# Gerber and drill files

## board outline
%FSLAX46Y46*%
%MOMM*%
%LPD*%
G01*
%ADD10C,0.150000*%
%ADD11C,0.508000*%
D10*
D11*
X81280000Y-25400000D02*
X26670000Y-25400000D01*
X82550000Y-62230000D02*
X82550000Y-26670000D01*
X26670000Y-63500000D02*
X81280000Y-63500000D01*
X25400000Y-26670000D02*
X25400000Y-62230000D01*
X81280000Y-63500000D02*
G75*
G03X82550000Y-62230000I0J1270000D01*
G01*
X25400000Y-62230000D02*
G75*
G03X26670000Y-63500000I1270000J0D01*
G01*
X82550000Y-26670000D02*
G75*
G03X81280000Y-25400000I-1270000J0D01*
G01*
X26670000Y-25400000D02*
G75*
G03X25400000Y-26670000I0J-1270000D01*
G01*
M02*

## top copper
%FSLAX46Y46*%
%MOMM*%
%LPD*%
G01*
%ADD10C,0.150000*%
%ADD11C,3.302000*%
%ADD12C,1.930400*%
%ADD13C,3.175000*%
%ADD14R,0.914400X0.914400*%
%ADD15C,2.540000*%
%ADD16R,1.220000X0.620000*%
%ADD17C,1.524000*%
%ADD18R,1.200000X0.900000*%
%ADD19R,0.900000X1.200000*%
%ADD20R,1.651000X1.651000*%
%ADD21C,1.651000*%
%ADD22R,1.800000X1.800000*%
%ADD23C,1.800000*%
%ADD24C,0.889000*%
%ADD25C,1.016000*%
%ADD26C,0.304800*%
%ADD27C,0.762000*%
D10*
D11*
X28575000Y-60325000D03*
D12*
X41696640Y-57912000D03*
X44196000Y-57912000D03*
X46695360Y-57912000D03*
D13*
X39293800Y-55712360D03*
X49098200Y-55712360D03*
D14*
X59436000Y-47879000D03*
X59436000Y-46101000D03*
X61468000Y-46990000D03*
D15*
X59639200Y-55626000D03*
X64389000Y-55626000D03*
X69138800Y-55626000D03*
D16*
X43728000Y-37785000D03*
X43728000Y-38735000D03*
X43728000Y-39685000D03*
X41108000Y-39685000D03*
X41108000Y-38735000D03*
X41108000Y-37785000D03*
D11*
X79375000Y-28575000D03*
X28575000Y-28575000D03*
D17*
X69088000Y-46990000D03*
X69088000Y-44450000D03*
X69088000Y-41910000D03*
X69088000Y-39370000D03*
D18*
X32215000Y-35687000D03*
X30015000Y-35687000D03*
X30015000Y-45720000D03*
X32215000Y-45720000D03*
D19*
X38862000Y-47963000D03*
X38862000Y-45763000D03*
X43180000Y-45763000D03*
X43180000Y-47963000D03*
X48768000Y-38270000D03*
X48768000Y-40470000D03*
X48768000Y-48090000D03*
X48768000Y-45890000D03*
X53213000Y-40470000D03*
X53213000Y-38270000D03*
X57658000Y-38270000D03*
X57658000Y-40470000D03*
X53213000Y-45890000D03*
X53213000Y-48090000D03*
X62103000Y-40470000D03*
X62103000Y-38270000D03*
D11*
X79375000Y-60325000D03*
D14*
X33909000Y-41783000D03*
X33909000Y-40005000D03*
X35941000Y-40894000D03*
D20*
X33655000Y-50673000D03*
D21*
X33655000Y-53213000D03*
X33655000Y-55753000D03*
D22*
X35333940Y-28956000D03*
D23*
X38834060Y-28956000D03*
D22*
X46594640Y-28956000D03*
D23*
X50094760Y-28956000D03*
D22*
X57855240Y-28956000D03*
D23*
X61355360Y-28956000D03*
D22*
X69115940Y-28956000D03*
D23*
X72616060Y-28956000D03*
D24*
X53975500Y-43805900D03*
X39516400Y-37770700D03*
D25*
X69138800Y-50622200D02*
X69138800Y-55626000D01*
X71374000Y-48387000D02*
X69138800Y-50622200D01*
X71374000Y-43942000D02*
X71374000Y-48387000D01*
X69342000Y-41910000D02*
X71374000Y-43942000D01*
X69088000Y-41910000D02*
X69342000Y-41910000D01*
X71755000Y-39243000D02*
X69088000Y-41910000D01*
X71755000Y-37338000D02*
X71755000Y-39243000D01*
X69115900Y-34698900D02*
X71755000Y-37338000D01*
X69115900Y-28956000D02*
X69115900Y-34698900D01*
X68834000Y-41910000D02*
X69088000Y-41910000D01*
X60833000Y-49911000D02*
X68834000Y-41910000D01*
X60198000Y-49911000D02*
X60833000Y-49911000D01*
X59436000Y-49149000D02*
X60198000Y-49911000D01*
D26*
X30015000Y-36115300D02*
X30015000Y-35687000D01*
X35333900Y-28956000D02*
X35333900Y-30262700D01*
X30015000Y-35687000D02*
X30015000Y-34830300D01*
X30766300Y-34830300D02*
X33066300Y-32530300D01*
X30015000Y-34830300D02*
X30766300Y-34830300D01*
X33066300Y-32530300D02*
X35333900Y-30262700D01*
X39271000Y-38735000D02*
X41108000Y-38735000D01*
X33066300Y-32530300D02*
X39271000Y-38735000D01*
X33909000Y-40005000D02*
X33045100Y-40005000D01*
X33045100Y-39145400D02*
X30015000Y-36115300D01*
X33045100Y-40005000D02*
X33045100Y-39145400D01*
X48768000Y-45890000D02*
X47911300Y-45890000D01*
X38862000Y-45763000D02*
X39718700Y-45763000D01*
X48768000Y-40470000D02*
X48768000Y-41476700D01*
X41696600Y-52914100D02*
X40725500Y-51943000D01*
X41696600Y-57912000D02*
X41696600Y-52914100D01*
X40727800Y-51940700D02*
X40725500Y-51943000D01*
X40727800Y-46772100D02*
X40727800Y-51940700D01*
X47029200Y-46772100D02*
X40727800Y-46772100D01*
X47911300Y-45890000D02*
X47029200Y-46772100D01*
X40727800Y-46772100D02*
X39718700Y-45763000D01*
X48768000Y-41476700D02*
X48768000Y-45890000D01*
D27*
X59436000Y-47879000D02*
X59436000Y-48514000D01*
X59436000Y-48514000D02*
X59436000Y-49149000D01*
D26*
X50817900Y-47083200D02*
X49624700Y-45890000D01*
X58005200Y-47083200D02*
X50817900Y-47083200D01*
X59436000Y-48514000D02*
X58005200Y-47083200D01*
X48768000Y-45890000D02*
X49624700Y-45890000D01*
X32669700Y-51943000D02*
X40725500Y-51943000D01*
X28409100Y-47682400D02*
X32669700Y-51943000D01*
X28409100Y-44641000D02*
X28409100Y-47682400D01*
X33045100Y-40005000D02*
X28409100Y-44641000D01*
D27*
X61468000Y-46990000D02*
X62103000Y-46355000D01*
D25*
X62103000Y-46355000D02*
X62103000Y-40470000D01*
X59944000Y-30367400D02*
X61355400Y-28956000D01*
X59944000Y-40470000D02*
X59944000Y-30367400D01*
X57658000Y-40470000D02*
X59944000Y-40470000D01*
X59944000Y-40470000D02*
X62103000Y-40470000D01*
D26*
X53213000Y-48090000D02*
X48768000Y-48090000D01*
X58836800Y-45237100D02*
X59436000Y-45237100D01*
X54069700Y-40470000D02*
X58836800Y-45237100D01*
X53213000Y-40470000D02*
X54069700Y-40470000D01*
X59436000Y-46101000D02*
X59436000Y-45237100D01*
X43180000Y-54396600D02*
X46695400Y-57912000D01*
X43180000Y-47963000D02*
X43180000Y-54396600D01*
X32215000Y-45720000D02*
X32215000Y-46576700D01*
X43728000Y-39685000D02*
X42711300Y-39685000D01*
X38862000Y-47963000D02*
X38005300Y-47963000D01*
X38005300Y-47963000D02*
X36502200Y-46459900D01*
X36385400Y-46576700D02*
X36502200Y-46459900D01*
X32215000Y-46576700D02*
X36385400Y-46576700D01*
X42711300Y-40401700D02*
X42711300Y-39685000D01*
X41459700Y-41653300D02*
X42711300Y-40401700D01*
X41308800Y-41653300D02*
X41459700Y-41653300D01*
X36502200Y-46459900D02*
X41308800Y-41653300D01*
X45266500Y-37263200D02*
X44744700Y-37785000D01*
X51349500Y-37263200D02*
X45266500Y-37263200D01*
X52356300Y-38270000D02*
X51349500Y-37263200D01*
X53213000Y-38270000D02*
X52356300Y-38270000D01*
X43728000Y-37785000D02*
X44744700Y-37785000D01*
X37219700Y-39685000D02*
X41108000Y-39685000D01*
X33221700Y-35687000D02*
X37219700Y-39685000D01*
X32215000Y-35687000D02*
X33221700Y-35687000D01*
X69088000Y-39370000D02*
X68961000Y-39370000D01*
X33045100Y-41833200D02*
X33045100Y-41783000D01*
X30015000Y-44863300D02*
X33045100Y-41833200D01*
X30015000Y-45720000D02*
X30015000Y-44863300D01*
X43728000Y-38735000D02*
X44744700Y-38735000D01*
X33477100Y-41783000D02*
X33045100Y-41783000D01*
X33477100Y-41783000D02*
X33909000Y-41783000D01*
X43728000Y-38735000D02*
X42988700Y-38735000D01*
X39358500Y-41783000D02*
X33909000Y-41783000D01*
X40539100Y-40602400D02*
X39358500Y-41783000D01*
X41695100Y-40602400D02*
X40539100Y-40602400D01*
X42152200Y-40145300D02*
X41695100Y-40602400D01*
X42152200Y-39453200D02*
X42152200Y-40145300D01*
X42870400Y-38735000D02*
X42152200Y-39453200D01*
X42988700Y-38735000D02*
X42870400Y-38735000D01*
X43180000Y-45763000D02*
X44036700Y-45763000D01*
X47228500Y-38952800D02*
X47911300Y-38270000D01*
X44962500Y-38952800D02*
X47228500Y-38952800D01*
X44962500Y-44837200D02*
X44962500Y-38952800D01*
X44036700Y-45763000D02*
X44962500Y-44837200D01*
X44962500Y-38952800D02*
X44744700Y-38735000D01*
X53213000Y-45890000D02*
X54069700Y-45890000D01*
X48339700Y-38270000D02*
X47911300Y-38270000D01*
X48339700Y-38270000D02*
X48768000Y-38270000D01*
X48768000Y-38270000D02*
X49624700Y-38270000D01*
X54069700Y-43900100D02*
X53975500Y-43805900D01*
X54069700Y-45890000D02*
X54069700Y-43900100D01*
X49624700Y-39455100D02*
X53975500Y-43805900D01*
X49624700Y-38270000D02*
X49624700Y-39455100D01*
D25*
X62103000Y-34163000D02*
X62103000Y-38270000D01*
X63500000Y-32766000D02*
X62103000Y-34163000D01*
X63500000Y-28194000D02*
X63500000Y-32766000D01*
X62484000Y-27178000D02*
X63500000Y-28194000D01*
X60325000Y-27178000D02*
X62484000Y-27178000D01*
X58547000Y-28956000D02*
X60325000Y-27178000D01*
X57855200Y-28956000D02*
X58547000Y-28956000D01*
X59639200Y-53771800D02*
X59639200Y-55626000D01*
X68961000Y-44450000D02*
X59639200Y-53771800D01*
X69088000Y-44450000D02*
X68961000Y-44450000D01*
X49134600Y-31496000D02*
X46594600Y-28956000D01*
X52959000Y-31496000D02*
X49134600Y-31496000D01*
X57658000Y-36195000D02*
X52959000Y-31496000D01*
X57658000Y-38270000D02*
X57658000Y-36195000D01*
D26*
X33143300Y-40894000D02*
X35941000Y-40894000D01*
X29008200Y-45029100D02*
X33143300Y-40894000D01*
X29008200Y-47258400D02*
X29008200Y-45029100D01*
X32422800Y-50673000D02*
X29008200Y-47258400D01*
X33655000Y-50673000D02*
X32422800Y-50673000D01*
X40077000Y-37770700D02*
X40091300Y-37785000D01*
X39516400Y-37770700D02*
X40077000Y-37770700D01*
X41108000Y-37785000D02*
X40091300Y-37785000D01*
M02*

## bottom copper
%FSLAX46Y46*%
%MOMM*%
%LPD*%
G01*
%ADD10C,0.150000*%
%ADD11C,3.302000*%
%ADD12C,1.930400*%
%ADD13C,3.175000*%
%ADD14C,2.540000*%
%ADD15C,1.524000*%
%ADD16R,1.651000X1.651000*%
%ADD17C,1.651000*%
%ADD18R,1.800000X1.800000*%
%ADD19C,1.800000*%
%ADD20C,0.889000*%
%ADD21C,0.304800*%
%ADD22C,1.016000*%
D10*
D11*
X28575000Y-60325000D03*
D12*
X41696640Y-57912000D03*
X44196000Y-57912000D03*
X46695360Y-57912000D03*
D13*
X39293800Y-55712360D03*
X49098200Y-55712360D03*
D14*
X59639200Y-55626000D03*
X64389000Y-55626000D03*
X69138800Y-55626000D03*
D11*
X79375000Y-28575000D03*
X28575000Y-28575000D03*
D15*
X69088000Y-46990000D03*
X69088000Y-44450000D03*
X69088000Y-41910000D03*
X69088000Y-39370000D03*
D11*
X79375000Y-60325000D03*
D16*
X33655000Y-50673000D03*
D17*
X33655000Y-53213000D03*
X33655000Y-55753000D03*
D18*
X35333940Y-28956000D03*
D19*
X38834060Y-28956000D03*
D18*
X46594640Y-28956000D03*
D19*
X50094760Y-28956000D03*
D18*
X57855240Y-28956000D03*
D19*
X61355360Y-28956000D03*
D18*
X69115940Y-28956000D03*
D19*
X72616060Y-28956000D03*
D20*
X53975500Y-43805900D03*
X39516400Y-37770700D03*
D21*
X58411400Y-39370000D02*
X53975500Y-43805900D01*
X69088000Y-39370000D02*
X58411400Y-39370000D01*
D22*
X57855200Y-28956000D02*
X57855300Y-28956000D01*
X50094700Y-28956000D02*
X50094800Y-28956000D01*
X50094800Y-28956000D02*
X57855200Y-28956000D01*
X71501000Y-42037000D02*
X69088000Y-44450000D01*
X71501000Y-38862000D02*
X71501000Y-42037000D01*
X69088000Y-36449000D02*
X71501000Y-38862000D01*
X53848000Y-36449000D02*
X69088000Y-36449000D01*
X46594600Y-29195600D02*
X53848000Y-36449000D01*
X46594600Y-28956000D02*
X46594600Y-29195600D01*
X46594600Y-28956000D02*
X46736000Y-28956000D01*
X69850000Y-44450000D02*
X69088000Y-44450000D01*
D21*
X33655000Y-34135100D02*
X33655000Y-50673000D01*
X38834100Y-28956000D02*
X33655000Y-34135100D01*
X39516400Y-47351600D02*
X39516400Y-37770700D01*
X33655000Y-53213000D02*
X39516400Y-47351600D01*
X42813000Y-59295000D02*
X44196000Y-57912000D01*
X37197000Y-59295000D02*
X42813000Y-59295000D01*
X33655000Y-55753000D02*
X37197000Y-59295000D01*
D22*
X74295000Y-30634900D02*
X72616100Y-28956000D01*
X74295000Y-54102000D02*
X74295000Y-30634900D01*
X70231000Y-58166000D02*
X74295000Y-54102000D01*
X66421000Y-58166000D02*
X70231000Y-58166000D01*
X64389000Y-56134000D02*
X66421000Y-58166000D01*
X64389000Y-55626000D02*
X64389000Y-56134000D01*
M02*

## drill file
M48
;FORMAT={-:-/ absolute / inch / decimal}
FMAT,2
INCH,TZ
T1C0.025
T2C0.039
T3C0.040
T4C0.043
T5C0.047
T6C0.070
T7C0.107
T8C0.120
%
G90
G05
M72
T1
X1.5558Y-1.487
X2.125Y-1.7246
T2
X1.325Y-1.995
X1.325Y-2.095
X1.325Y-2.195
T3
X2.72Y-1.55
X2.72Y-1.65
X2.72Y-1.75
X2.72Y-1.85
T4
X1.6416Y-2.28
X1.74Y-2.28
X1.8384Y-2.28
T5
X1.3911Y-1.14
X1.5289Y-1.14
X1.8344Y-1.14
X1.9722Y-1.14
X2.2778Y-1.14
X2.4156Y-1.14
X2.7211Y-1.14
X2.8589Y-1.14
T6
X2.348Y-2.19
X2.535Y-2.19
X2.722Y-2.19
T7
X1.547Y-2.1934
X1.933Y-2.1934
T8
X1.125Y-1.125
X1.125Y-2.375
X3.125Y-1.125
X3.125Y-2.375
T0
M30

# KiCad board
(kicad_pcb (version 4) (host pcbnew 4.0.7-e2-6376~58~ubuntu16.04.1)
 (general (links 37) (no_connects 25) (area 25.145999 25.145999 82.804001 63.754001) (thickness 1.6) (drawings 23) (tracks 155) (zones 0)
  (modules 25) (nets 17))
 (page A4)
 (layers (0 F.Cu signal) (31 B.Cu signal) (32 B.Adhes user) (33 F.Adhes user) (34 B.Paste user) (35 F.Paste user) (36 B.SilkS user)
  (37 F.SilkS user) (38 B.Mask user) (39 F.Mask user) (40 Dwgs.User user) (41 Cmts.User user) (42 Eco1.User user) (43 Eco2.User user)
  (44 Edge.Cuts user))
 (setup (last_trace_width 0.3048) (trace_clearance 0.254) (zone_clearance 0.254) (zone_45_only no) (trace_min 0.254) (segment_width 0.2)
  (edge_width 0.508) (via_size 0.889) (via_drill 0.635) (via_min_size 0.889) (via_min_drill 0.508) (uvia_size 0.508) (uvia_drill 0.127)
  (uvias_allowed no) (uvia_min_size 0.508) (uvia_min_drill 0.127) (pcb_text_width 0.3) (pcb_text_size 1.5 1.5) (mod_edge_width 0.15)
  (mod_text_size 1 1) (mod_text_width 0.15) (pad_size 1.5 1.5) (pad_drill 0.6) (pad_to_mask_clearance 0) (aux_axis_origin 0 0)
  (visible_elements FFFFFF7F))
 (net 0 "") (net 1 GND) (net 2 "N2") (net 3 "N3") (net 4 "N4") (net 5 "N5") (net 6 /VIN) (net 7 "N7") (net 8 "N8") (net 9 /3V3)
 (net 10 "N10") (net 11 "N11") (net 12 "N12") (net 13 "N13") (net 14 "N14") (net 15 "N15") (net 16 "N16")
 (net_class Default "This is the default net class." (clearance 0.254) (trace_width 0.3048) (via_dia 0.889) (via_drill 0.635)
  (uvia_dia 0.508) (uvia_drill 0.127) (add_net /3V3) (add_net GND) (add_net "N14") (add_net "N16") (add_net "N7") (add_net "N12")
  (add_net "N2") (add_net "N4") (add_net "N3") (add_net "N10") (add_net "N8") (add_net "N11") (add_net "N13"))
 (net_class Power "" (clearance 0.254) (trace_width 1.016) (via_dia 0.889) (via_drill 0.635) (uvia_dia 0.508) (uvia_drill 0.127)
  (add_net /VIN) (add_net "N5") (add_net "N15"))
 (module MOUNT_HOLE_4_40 (layer F.Cu) (at 38.608 53.34)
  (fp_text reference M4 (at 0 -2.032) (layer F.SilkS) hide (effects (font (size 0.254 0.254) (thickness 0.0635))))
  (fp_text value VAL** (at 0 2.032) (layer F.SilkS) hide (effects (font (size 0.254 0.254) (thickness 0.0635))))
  (pad "" thru_hole circle (at -10.033 6.985) (size 3.302 3.302) (drill 3.048) (layers *.Cu *.SilkS *.Mask)))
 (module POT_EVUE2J (layer F.Cu) (at 44.196 57.912 270)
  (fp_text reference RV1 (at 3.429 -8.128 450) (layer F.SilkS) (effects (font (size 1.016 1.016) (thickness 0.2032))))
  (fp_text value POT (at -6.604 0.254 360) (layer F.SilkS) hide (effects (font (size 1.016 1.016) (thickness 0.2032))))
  (pad 1 thru_hole circle (at 0 2.49936 270) (size 1.9304 1.9304) (drill 1.09982) (layers *.Cu *.Mask F.SilkS) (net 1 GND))
  (pad 2 thru_hole circle (at 0 0 270) (size 1.9304 1.9304) (drill 1.09982) (layers *.Cu *.Mask F.SilkS) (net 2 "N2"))
  (pad 3 thru_hole circle (at 0 -2.49936 270) (size 1.9304 1.9304) (drill 1.09982) (layers *.Cu *.Mask F.SilkS) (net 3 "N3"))
  (pad "" thru_hole circle (at -2.19964 4.9022 270) (size 3.175 3.175) (drill 2.7178) (layers *.Cu *.Mask F.SilkS))
  (pad "" thru_hole circle (at -2.19964 -4.9022 270) (size 3.175 3.175) (drill 2.7178) (layers *.Cu *.Mask F.SilkS)))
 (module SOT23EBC (layer F.Cu) (at 60.452 46.99 90)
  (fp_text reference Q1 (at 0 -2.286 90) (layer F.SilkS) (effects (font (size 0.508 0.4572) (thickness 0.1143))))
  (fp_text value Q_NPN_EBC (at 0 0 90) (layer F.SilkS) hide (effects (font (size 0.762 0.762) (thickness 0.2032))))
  (pad 1 smd rect (at -0.889 -1.016 90) (size 0.9144 0.9144) (layers F.Cu F.Paste F.Mask) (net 1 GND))
  (pad 2 smd rect (at 0.889 -1.016 90) (size 0.9144 0.9144) (layers F.Cu F.Paste F.Mask) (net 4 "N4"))
  (pad 3 smd rect (at 0 1.016 90) (size 0.9144 0.9144) (layers F.Cu F.Paste F.Mask) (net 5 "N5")))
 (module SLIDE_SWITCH (layer F.Cu) (at 64.389 58.166)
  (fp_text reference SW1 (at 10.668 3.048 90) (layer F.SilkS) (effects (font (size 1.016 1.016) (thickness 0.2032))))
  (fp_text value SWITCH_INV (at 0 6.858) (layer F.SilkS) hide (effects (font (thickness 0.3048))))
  (pad 1 thru_hole circle (at -4.7498 -2.54) (size 2.54 2.54) (drill 1.778) (layers *.Cu *.Mask F.SilkS) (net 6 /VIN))
  (pad 2 thru_hole circle (at 0 -2.54) (size 2.54 2.54) (drill 1.778) (layers *.Cu *.Mask F.SilkS) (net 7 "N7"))
  (pad 3 thru_hole circle (at 4.7498 -2.54) (size 2.54 2.54) (drill 1.778) (layers *.Cu *.Mask F.SilkS) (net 1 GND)))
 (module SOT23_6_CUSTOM (layer F.Cu) (at 42.418 38.735 270)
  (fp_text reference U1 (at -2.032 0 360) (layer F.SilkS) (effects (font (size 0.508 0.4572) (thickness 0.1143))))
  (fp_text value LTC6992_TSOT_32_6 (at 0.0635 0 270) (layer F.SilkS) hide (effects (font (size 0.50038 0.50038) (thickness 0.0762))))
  (pad 6 smd rect (at -0.95 -1.31 270) (size 0.62 1.22) (layers F.Cu F.Paste F.Mask) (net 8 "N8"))
  (pad 5 smd rect (at 0 -1.31 270) (size 0.62 1.22) (layers F.Cu F.Paste F.Mask) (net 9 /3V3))
  (pad 4 smd rect (at 0.95 -1.31 270) (size 0.62 1.22) (layers F.Cu F.Paste F.Mask) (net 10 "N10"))
  (pad 3 smd rect (at 0.95 1.31 270) (size 0.62 1.22) (layers F.Cu F.Paste F.Mask) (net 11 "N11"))
  (pad 2 smd rect (at 0 1.31 270) (size 0.62 1.22) (layers F.Cu F.Paste F.Mask) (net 1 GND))
  (pad 1 smd rect (at -0.95 1.31 270) (size 0.62 1.22) (layers F.Cu F.Paste F.Mask) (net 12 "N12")))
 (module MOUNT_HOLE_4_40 (layer F.Cu) (at 100.965 20.955)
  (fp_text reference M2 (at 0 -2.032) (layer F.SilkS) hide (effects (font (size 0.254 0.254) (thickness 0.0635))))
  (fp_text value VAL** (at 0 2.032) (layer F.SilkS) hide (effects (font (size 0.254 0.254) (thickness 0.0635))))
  (pad "" thru_hole circle (at -21.59 7.62) (size 3.302 3.302) (drill 3.048) (layers *.Cu *.SilkS *.Mask)))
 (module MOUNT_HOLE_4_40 (layer F.Cu) (at 28.575 28.575)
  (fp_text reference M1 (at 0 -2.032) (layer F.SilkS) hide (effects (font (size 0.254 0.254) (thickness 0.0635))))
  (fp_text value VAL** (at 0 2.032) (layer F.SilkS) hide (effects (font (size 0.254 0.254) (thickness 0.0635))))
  (pad "" thru_hole circle (at 0 0) (size 3.302 3.302) (drill 3.048) (layers *.Cu *.SilkS *.Mask)))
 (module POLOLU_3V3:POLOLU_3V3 (layer F.Cu) (at 69.088 43.18 90)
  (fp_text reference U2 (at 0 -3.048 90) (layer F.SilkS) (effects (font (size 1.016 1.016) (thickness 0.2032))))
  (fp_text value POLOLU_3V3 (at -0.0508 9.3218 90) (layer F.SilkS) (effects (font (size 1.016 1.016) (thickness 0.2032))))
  (pad 1 thru_hole circle (at -3.81 0 90) (size 1.524 1.524) (drill 1.016) (layers *.Cu *.Mask F.SilkS) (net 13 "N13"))
  (pad 2 thru_hole circle (at -1.27 0 90) (size 1.524 1.524) (drill 1.016) (layers *.Cu *.Mask F.SilkS) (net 6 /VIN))
  (pad 3 thru_hole circle (at 1.27 0 90) (size 1.524 1.524) (drill 1.016) (layers *.Cu *.Mask F.SilkS) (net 1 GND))
  (pad 4 thru_hole circle (at 3.81 0 90) (size 1.524 1.524) (drill 1.016) (layers *.Cu *.Mask F.SilkS) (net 9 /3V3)))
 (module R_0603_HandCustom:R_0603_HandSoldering (layer F.Cu) (at 31.115 35.687 180)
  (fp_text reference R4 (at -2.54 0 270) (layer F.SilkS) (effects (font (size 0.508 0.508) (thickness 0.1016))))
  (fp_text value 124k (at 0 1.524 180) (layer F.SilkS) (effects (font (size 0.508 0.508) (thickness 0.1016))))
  (pad 1 smd rect (at -1.1 0 180) (size 1.2 0.9) (layers F.Cu F.Paste F.Mask) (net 11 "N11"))
  (pad 2 smd rect (at 1.1 0 180) (size 1.2 0.9) (layers F.Cu F.Paste F.Mask) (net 1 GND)))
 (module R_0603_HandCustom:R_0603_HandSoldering (layer F.Cu) (at 31.115 45.72)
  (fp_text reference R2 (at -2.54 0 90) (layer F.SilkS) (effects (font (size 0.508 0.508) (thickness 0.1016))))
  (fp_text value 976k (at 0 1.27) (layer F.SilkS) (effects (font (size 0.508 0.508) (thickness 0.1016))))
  (pad 1 smd rect (at -1.1 0) (size 1.2 0.9) (layers F.Cu F.Paste F.Mask) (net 9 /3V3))
  (pad 2 smd rect (at 1.1 0) (size 1.2 0.9) (layers F.Cu F.Paste F.Mask) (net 10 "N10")))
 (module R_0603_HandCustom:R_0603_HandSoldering (layer F.Cu) (at 38.862 46.863 90)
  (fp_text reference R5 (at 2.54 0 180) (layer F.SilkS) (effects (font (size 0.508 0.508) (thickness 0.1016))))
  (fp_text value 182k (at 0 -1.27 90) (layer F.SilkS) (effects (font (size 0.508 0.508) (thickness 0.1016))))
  (pad 1 smd rect (at -1.1 0 90) (size 1.2 0.9) (layers F.Cu F.Paste F.Mask) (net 10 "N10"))
  (pad 2 smd rect (at 1.1 0 90) (size 1.2 0.9) (layers F.Cu F.Paste F.Mask) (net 1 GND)))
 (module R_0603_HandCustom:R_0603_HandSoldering (layer F.Cu) (at 43.18 46.863 270)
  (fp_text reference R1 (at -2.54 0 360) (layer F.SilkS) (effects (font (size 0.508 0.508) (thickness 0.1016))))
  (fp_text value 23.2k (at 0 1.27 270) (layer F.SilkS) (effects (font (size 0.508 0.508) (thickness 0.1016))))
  (pad 1 smd rect (at -1.1 0 270) (size 1.2 0.9) (layers F.Cu F.Paste F.Mask) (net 9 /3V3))
  (pad 2 smd rect (at 1.1 0 270) (size 1.2 0.9) (layers F.Cu F.Paste F.Mask) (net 3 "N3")))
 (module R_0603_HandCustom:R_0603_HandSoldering (layer F.Cu) (at 48.768 39.37 270)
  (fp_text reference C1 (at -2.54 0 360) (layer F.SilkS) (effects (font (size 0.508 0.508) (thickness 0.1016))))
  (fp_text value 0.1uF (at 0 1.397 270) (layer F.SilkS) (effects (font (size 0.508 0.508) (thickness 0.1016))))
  (pad 1 smd rect (at -1.1 0 270) (size 1.2 0.9) (layers F.Cu F.Paste F.Mask) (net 9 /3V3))
  (pad 2 smd rect (at 1.1 0 270) (size 1.2 0.9) (layers F.Cu F.Paste F.Mask) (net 1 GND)))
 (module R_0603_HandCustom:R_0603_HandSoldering (layer F.Cu) (at 48.768 46.99 90)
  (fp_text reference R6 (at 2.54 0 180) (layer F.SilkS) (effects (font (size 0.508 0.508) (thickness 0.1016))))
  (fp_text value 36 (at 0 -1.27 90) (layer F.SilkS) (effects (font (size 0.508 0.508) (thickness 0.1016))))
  (pad 1 smd rect (at -1.1 0 90) (size 1.2 0.9) (layers F.Cu F.Paste F.Mask) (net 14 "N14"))
  (pad 2 smd rect (at 1.1 0 90) (size 1.2 0.9) (layers F.Cu F.Paste F.Mask) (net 1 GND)))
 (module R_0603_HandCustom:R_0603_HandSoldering (layer F.Cu) (at 53.213 39.37 90)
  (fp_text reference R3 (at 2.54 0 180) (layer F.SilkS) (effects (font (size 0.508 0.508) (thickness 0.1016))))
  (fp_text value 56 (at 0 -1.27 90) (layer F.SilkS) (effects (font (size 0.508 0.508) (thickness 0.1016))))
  (pad 1 smd rect (at -1.1 0 90) (size 1.2 0.9) (layers F.Cu F.Paste F.Mask) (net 4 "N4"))
  (pad 2 smd rect (at 1.1 0 90) (size 1.2 0.9) (layers F.Cu F.Paste F.Mask) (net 8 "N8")))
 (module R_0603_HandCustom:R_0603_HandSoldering (layer F.Cu) (at 57.658 39.37 270)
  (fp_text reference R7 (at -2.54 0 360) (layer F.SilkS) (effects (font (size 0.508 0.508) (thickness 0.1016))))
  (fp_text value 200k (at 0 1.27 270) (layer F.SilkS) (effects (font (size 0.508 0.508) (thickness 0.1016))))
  (pad 1 smd rect (at -1.1 0 270) (size 1.2 0.9) (layers F.Cu F.Paste F.Mask) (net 6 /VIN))
  (pad 2 smd rect (at 1.1 0 270) (size 1.2 0.9) (layers F.Cu F.Paste F.Mask) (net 5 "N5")))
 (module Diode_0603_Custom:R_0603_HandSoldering (layer F.Cu) (at 53.213 46.99 270)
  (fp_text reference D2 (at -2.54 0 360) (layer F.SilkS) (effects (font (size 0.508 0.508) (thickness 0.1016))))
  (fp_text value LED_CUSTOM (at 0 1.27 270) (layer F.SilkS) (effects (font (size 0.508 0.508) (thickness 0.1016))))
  (pad 1 smd rect (at -1.1 0 270) (size 1.2 0.9) (layers F.Cu F.Paste F.Mask) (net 9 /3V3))
  (pad 2 smd rect (at 1.1 0 270) (size 1.2 0.9) (layers F.Cu F.Paste F.Mask) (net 14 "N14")))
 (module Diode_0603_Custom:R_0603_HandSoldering (layer F.Cu) (at 62.103 39.37 90)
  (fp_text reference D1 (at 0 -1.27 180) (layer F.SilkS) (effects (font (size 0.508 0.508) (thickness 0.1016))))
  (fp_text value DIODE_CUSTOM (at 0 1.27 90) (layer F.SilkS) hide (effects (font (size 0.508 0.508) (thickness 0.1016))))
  (pad 1 smd rect (at -1.1 0 90) (size 1.2 0.9) (layers F.Cu F.Paste F.Mask) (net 5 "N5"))
  (pad 2 smd rect (at 1.1 0 90) (size 1.2 0.9) (layers F.Cu F.Paste F.Mask) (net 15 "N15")))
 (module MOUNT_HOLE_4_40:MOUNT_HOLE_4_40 (layer F.Cu) (at 79.375 60.325)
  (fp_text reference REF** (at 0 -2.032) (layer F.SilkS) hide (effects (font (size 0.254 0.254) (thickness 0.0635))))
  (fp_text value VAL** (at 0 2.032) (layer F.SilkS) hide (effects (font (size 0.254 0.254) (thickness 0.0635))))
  (pad "" thru_hole circle (at 0 0) (size 3.302 3.302) (drill 3.048) (layers *.Cu *.SilkS *.Mask)))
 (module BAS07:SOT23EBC (layer F.Cu) (at 33.909 40.894 270)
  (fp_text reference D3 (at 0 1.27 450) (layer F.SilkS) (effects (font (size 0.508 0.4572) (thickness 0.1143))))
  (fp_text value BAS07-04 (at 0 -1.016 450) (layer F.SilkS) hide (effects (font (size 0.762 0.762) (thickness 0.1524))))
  (pad 2 smd rect (at 0.889 0 90) (size 0.9144 0.9144) (layers F.Cu F.Paste F.Mask) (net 9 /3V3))
  (pad 1 smd rect (at -0.889 0 90) (size 0.9144 0.9144) (layers F.Cu F.Paste F.Mask) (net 1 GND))
  (pad 3 smd rect (at 0 -2.032 90) (size 0.9144 0.9144) (layers F.Cu F.Paste F.Mask) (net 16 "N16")))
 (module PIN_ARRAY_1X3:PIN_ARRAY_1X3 (layer F.Cu) (at 33.655 53.213)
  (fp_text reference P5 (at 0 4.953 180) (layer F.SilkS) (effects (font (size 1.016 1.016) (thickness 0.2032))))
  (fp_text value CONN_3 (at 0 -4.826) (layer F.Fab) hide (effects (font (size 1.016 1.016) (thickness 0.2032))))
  (pad 1 thru_hole rect (at 0 -2.54) (size 1.651 1.651) (drill 0.9906) (layers *.Cu *.Mask) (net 16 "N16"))
  (pad 2 thru_hole circle (at 0 0) (size 1.651 1.651) (drill 0.9906) (layers *.Cu *.Mask) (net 12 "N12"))
  (pad 3 thru_hole circle (at 0 2.54) (size 1.651 1.651) (drill 0.9906) (layers *.Cu *.Mask) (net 2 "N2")))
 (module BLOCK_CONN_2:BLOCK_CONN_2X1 (layer F.Cu) (at 37.084 28.956)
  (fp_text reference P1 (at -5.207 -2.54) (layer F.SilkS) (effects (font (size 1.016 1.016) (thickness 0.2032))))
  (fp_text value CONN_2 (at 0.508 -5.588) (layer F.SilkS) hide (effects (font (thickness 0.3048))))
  (pad 1 thru_hole rect (at -1.75006 0) (size 1.8 1.8) (drill 1.2) (layers *.Cu *.Mask F.SilkS) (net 1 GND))
  (pad 2 thru_hole circle (at 1.75006 0) (size 1.8 1.8) (drill 1.2) (layers *.Cu *.Mask F.SilkS) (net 16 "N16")))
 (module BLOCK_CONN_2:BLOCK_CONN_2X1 (layer F.Cu) (at 48.3447 28.956)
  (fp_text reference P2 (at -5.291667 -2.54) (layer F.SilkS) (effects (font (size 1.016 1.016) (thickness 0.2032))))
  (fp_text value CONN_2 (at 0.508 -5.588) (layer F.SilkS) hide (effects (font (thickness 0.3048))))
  (pad 1 thru_hole rect (at -1.75006 0) (size 1.8 1.8) (drill 1.2) (layers *.Cu *.Mask F.SilkS) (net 6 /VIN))
  (pad 2 thru_hole circle (at 1.75006 0) (size 1.8 1.8) (drill 1.2) (layers *.Cu *.Mask F.SilkS) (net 15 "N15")))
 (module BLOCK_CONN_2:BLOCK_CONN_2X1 (layer F.Cu) (at 59.6053 28.956)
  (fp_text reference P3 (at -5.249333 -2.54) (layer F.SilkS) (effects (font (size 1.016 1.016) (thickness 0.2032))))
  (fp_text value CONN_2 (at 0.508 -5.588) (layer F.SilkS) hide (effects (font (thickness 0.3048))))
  (pad 1 thru_hole rect (at -1.75006 0) (size 1.8 1.8) (drill 1.2) (layers *.Cu *.Mask F.SilkS) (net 15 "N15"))
  (pad 2 thru_hole circle (at 1.75006 0) (size 1.8 1.8) (drill 1.2) (layers *.Cu *.Mask F.SilkS) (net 5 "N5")))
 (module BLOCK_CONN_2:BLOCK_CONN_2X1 (layer F.Cu) (at 70.866 28.956)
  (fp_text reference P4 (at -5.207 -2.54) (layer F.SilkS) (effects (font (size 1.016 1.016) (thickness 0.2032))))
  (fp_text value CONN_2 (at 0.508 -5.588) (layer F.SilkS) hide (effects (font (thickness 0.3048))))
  (pad 1 thru_hole rect (at -1.75006 0) (size 1.8 1.8) (drill 1.2) (layers *.Cu *.Mask F.SilkS) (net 1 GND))
  (pad 2 thru_hole circle (at 1.75006 0) (size 1.8 1.8) (drill 1.2) (layers *.Cu *.Mask F.SilkS) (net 7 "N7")))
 (gr_line (start 81.28 25.4) (end 26.67 25.4) (angle 90) (layer Edge.Cuts) (width 0.508))
 (gr_line (start 82.55 62.23) (end 82.55 26.67) (angle 90) (layer Edge.Cuts) (width 0.508))
 (gr_line (start 26.67 63.5) (end 81.28 63.5) (angle 90) (layer Edge.Cuts) (width 0.508))
 (gr_line (start 25.4 26.67) (end 25.4 62.23) (angle 90) (layer Edge.Cuts) (width 0.508))
 (gr_arc (start 81.28 62.23) (end 82.55 62.23) (angle 90) (layer Edge.Cuts) (width 0.508))
 (gr_arc (start 26.67 62.23) (end 26.67 63.5) (angle 90) (layer Edge.Cuts) (width 0.508))
 (gr_arc (start 81.28 26.67) (end 81.28 25.4) (angle 90) (layer Edge.Cuts) (width 0.508))
 (gr_arc (start 26.67 26.67) (end 25.4 26.67) (angle 90) (layer Edge.Cuts) (width 0.508))
 (segment (start 69.1388 50.6222) (end 69.1388 55.626) (width 1.016) (layer F.Cu) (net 1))
 (segment (start 71.374 48.387) (end 69.1388 50.6222) (width 1.016) (layer F.Cu) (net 1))
 (segment (start 71.374 43.942) (end 71.374 48.387) (width 1.016) (layer F.Cu) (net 1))
 (segment (start 69.342 41.91) (end 71.374 43.942) (width 1.016) (layer F.Cu) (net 1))
 (segment (start 69.088 41.91) (end 69.342 41.91) (width 1.016) (layer F.Cu) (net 1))
 (segment (start 71.755 39.243) (end 69.088 41.91) (width 1.016) (layer F.Cu) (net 1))
 (segment (start 71.755 37.338) (end 71.755 39.243) (width 1.016) (layer F.Cu) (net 1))
 (segment (start 69.1159 34.6989) (end 71.755 37.338) (width 1.016) (layer F.Cu) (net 1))
 (segment (start 69.1159 28.956) (end 69.1159 34.6989) (width 1.016) (layer F.Cu) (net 1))
 (segment (start 68.834 41.91) (end 69.088 41.91) (width 1.016) (layer F.Cu) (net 1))
 (segment (start 60.833 49.911) (end 68.834 41.91) (width 1.016) (layer F.Cu) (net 1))
 (segment (start 60.198 49.911) (end 60.833 49.911) (width 1.016) (layer F.Cu) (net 1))
 (segment (start 59.436 49.149) (end 60.198 49.911) (width 1.016) (layer F.Cu) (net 1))
 (segment (start 30.015 36.1153) (end 30.015 35.687) (width 0.3048) (layer F.Cu) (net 1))
 (segment (start 35.3339 28.956) (end 35.3339 30.2627) (width 0.3048) (layer F.Cu) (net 1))
 (segment (start 30.015 35.687) (end 30.015 34.8303) (width 0.3048) (layer F.Cu) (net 1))
 (segment (start 30.7663 34.8303) (end 33.0663 32.5303) (width 0.3048) (layer F.Cu) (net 1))
 (segment (start 30.015 34.8303) (end 30.7663 34.8303) (width 0.3048) (layer F.Cu) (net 1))
 (segment (start 33.0663 32.5303) (end 35.3339 30.2627) (width 0.3048) (layer F.Cu) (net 1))
 (segment (start 39.271 38.735) (end 41.108 38.735) (width 0.3048) (layer F.Cu) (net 1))
 (segment (start 33.0663 32.5303) (end 39.271 38.735) (width 0.3048) (layer F.Cu) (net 1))
 (segment (start 33.909 40.005) (end 33.0451 40.005) (width 0.3048) (layer F.Cu) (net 1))
 (segment (start 33.0451 39.1454) (end 30.015 36.1153) (width 0.3048) (layer F.Cu) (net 1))
 (segment (start 33.0451 40.005) (end 33.0451 39.1454) (width 0.3048) (layer F.Cu) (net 1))
 (segment (start 48.768 45.89) (end 47.9113 45.89) (width 0.3048) (layer F.Cu) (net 1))
 (segment (start 38.862 45.763) (end 39.7187 45.763) (width 0.3048) (layer F.Cu) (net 1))
 (segment (start 48.768 40.47) (end 48.768 41.4767) (width 0.3048) (layer F.Cu) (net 1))
 (segment (start 41.6966 52.9141) (end 40.7255 51.943) (width 0.3048) (layer F.Cu) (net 1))
 (segment (start 41.6966 57.912) (end 41.6966 52.9141) (width 0.3048) (layer F.Cu) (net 1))
 (segment (start 40.7278 51.9407) (end 40.7255 51.943) (width 0.3048) (layer F.Cu) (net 1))
 (segment (start 40.7278 46.7721) (end 40.7278 51.9407) (width 0.3048) (layer F.Cu) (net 1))
 (segment (start 47.0292 46.7721) (end 40.7278 46.7721) (width 0.3048) (layer F.Cu) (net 1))
 (segment (start 47.9113 45.89) (end 47.0292 46.7721) (width 0.3048) (layer F.Cu) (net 1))
 (segment (start 40.7278 46.7721) (end 39.7187 45.763) (width 0.3048) (layer F.Cu) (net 1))
 (segment (start 48.768 41.4767) (end 48.768 45.89) (width 0.3048) (layer F.Cu) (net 1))
 (segment (start 59.436 47.879) (end 59.436 48.514) (width 0.762) (layer F.Cu) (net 1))
 (segment (start 59.436 48.514) (end 59.436 49.149) (width 0.762) (layer F.Cu) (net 1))
 (segment (start 50.8179 47.0832) (end 49.6247 45.89) (width 0.3048) (layer F.Cu) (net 1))
 (segment (start 58.0052 47.0832) (end 50.8179 47.0832) (width 0.3048) (layer F.Cu) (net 1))
 (segment (start 59.436 48.514) (end 58.0052 47.0832) (width 0.3048) (layer F.Cu) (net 1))
 (segment (start 48.768 45.89) (end 49.6247 45.89) (width 0.3048) (layer F.Cu) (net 1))
 (segment (start 32.6697 51.943) (end 40.7255 51.943) (width 0.3048) (layer F.Cu) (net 1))
 (segment (start 28.4091 47.6824) (end 32.6697 51.943) (width 0.3048) (layer F.Cu) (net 1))
 (segment (start 28.4091 44.641) (end 28.4091 47.6824) (width 0.3048) (layer F.Cu) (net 1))
 (segment (start 33.0451 40.005) (end 28.4091 44.641) (width 0.3048) (layer F.Cu) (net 1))
 (segment (start 61.468 46.99) (end 62.103 46.355) (width 0.762) (layer F.Cu) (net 5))
 (segment (start 62.103 46.355) (end 62.103 40.47) (width 1.016) (layer F.Cu) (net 5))
 (segment (start 59.944 30.3674) (end 61.3554 28.956) (width 1.016) (layer F.Cu) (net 5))
 (segment (start 59.944 40.47) (end 59.944 30.3674) (width 1.016) (layer F.Cu) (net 5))
 (segment (start 57.658 40.47) (end 59.944 40.47) (width 1.016) (layer F.Cu) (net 5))
 (segment (start 59.944 40.47) (end 62.103 40.47) (width 1.016) (layer F.Cu) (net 5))
 (segment (start 53.213 48.09) (end 48.768 48.09) (width 0.3048) (layer F.Cu) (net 14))
 (segment (start 58.8368 45.2371) (end 59.436 45.2371) (width 0.3048) (layer F.Cu) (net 4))
 (segment (start 54.0697 40.47) (end 58.8368 45.2371) (width 0.3048) (layer F.Cu) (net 4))
 (segment (start 53.213 40.47) (end 54.0697 40.47) (width 0.3048) (layer F.Cu) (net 4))
 (segment (start 59.436 46.101) (end 59.436 45.2371) (width 0.3048) (layer F.Cu) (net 4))
 (segment (start 43.18 54.3966) (end 46.6954 57.912) (width 0.3048) (layer F.Cu) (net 3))
 (segment (start 43.18 47.963) (end 43.18 54.3966) (width 0.3048) (layer F.Cu) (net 3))
 (segment (start 32.215 45.72) (end 32.215 46.5767) (width 0.3048) (layer F.Cu) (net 10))
 (segment (start 43.728 39.685) (end 42.7113 39.685) (width 0.3048) (layer F.Cu) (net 10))
 (segment (start 38.862 47.963) (end 38.0053 47.963) (width 0.3048) (layer F.Cu) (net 10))
 (segment (start 38.0053 47.963) (end 36.5022 46.4599) (width 0.3048) (layer F.Cu) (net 10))
 (segment (start 36.3854 46.5767) (end 36.5022 46.4599) (width 0.3048) (layer F.Cu) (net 10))
 (segment (start 32.215 46.5767) (end 36.3854 46.5767) (width 0.3048) (layer F.Cu) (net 10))
 (segment (start 42.7113 40.4017) (end 42.7113 39.685) (width 0.3048) (layer F.Cu) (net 10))
 (segment (start 41.4597 41.6533) (end 42.7113 40.4017) (width 0.3048) (layer F.Cu) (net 10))
 (segment (start 41.3088 41.6533) (end 41.4597 41.6533) (width 0.3048) (layer F.Cu) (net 10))
 (segment (start 36.5022 46.4599) (end 41.3088 41.6533) (width 0.3048) (layer F.Cu) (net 10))
 (segment (start 45.2665 37.2632) (end 44.7447 37.785) (width 0.3048) (layer F.Cu) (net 8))
 (segment (start 51.3495 37.2632) (end 45.2665 37.2632) (width 0.3048) (layer F.Cu) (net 8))
 (segment (start 52.3563 38.27) (end 51.3495 37.2632) (width 0.3048) (layer F.Cu) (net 8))
 (segment (start 53.213 38.27) (end 52.3563 38.27) (width 0.3048) (layer F.Cu) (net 8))
 (segment (start 43.728 37.785) (end 44.7447 37.785) (width 0.3048) (layer F.Cu) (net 8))
 (segment (start 37.2197 39.685) (end 41.108 39.685) (width 0.3048) (layer F.Cu) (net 11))
 (segment (start 33.2217 35.687) (end 37.2197 39.685) (width 0.3048) (layer F.Cu) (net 11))
 (segment (start 32.215 35.687) (end 33.2217 35.687) (width 0.3048) (layer F.Cu) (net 11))
 (via (at 53.9755 43.8059) (size 0.889) (layers F.Cu B.Cu) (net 9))
 (segment (start 69.088 39.37) (end 68.961 39.37) (width 0.3048) (layer F.Cu) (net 9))
 (segment (start 33.0451 41.8332) (end 33.0451 41.783) (width 0.3048) (layer F.Cu) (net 9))
 (segment (start 30.015 44.8633) (end 33.0451 41.8332) (width 0.3048) (layer F.Cu) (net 9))
 (segment (start 30.015 45.72) (end 30.015 44.8633) (width 0.3048) (layer F.Cu) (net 9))
 (segment (start 43.728 38.735) (end 44.7447 38.735) (width 0.3048) (layer F.Cu) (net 9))
 (segment (start 33.4771 41.783) (end 33.0451 41.783) (width 0.3048) (layer F.Cu) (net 9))
 (segment (start 33.4771 41.783) (end 33.909 41.783) (width 0.3048) (layer F.Cu) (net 9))
 (segment (start 43.728 38.735) (end 42.9887 38.735) (width 0.3048) (layer F.Cu) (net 9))
 (segment (start 39.3585 41.783) (end 33.909 41.783) (width 0.3048) (layer F.Cu) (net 9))
 (segment (start 40.5391 40.6024) (end 39.3585 41.783) (width 0.3048) (layer F.Cu) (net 9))
 (segment (start 41.6951 40.6024) (end 40.5391 40.6024) (width 0.3048) (layer F.Cu) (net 9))
 (segment (start 42.1522 40.1453) (end 41.6951 40.6024) (width 0.3048) (layer F.Cu) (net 9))
 (segment (start 42.1522 39.4532) (end 42.1522 40.1453) (width 0.3048) (layer F.Cu) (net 9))
 (segment (start 42.8704 38.735) (end 42.1522 39.4532) (width 0.3048) (layer F.Cu) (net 9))
 (segment (start 42.9887 38.735) (end 42.8704 38.735) (width 0.3048) (layer F.Cu) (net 9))
 (segment (start 43.18 45.763) (end 44.0367 45.763) (width 0.3048) (layer F.Cu) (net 9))
 (segment (start 47.2285 38.9528) (end 47.9113 38.27) (width 0.3048) (layer F.Cu) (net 9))
 (segment (start 44.9625 38.9528) (end 47.2285 38.9528) (width 0.3048) (layer F.Cu) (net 9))
 (segment (start 44.9625 44.8372) (end 44.9625 38.9528) (width 0.3048) (layer F.Cu) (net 9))
 (segment (start 44.0367 45.763) (end 44.9625 44.8372) (width 0.3048) (layer F.Cu) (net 9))
 (segment (start 44.9625 38.9528) (end 44.7447 38.735) (width 0.3048) (layer F.Cu) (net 9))
 (segment (start 53.213 45.89) (end 54.0697 45.89) (width 0.3048) (layer F.Cu) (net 9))
 (segment (start 48.3397 38.27) (end 47.9113 38.27) (width 0.3048) (layer F.Cu) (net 9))
 (segment (start 48.3397 38.27) (end 48.768 38.27) (width 0.3048) (layer F.Cu) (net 9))
 (segment (start 48.768 38.27) (end 49.6247 38.27) (width 0.3048) (layer F.Cu) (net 9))
 (segment (start 58.4114 39.37) (end 53.9755 43.8059) (width 0.3048) (layer B.Cu) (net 9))
 (segment (start 69.088 39.37) (end 58.4114 39.37) (width 0.3048) (layer B.Cu) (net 9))
 (segment (start 54.0697 43.9001) (end 53.9755 43.8059) (width 0.3048) (layer F.Cu) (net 9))
 (segment (start 54.0697 45.89) (end 54.0697 43.9001) (width 0.3048) (layer F.Cu) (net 9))
 (segment (start 49.6247 39.4551) (end 53.9755 43.8059) (width 0.3048) (layer F.Cu) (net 9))
 (segment (start 49.6247 38.27) (end 49.6247 39.4551) (width 0.3048) (layer F.Cu) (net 9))
 (segment (start 57.8552 28.956) (end 57.8553 28.956) (width 1.016) (layer B.Cu) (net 15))
 (segment (start 62.103 34.163) (end 62.103 38.27) (width 1.016) (layer F.Cu) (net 15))
 (segment (start 63.5 32.766) (end 62.103 34.163) (width 1.016) (layer F.Cu) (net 15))
 (segment (start 63.5 28.194) (end 63.5 32.766) (width 1.016) (layer F.Cu) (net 15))
 (segment (start 62.484 27.178) (end 63.5 28.194) (width 1.016) (layer F.Cu) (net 15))
 (segment (start 60.325 27.178) (end 62.484 27.178) (width 1.016) (layer F.Cu) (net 15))
 (segment (start 58.547 28.956) (end 60.325 27.178) (width 1.016) (layer F.Cu) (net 15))
 (segment (start 57.8552 28.956) (end 58.547 28.956) (width 1.016) (layer F.Cu) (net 15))
 (segment (start 50.0947 28.956) (end 50.0948 28.956) (width 1.016) (layer B.Cu) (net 15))
 (segment (start 50.0948 28.956) (end 57.8552 28.956) (width 1.016) (layer B.Cu) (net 15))
 (segment (start 71.501 42.037) (end 69.088 44.45) (width 1.016) (layer B.Cu) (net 6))
 (segment (start 71.501 38.862) (end 71.501 42.037) (width 1.016) (layer B.Cu) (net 6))
 (segment (start 69.088 36.449) (end 71.501 38.862) (width 1.016) (layer B.Cu) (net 6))
 (segment (start 53.848 36.449) (end 69.088 36.449) (width 1.016) (layer B.Cu) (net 6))
 (segment (start 46.5946 29.1956) (end 53.848 36.449) (width 1.016) (layer B.Cu) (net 6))
 (segment (start 46.5946 28.956) (end 46.5946 29.1956) (width 1.016) (layer B.Cu) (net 6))
 (segment (start 46.5946 28.956) (end 46.736 28.956) (width 1.016) (layer B.Cu) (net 6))
 (segment (start 69.85 44.45) (end 69.088 44.45) (width 1.016) (layer B.Cu) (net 6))
 (segment (start 59.6392 53.7718) (end 59.6392 55.626) (width 1.016) (layer F.Cu) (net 6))
 (segment (start 68.961 44.45) (end 59.6392 53.7718) (width 1.016) (layer F.Cu) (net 6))
 (segment (start 69.088 44.45) (end 68.961 44.45) (width 1.016) (layer F.Cu) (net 6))
 (segment (start 49.1346 31.496) (end 46.5946 28.956) (width 1.016) (layer F.Cu) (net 6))
 (segment (start 52.959 31.496) (end 49.1346 31.496) (width 1.016) (layer F.Cu) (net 6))
 (segment (start 57.658 36.195) (end 52.959 31.496) (width 1.016) (layer F.Cu) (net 6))
 (segment (start 57.658 38.27) (end 57.658 36.195) (width 1.016) (layer F.Cu) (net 6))
 (segment (start 33.655 34.1351) (end 33.655 50.673) (width 0.3048) (layer B.Cu) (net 16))
 (segment (start 38.8341 28.956) (end 33.655 34.1351) (width 0.3048) (layer B.Cu) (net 16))
 (segment (start 33.1433 40.894) (end 35.941 40.894) (width 0.3048) (layer F.Cu) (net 16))
 (segment (start 29.0082 45.0291) (end 33.1433 40.894) (width 0.3048) (layer F.Cu) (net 16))
 (segment (start 29.0082 47.2584) (end 29.0082 45.0291) (width 0.3048) (layer F.Cu) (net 16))
 (segment (start 32.4228 50.673) (end 29.0082 47.2584) (width 0.3048) (layer F.Cu) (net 16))
 (segment (start 33.655 50.673) (end 32.4228 50.673) (width 0.3048) (layer F.Cu) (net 16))
 (via (at 39.5164 37.7707) (size 0.889) (layers F.Cu B.Cu) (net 12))
 (segment (start 39.5164 47.3516) (end 39.5164 37.7707) (width 0.3048) (layer B.Cu) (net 12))
 (segment (start 33.655 53.213) (end 39.5164 47.3516) (width 0.3048) (layer B.Cu) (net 12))
 (segment (start 40.077 37.7707) (end 40.0913 37.785) (width 0.3048) (layer F.Cu) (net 12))
 (segment (start 39.5164 37.7707) (end 40.077 37.7707) (width 0.3048) (layer F.Cu) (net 12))
 (segment (start 41.108 37.785) (end 40.0913 37.785) (width 0.3048) (layer F.Cu) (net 12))
 (segment (start 42.813 59.295) (end 44.196 57.912) (width 0.3048) (layer B.Cu) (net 2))
 (segment (start 37.197 59.295) (end 42.813 59.295) (width 0.3048) (layer B.Cu) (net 2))
 (segment (start 33.655 55.753) (end 37.197 59.295) (width 0.3048) (layer B.Cu) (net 2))
 (segment (start 74.295 30.6349) (end 72.6161 28.956) (width 1.016) (layer B.Cu) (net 7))
 (segment (start 74.295 54.102) (end 74.295 30.6349) (width 1.016) (layer B.Cu) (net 7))
 (segment (start 70.231 58.166) (end 74.295 54.102) (width 1.016) (layer B.Cu) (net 7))
 (segment (start 66.421 58.166) (end 70.231 58.166) (width 1.016) (layer B.Cu) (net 7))
 (segment (start 64.389 56.134) (end 66.421 58.166) (width 1.016) (layer B.Cu) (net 7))
 (segment (start 64.389 55.626) (end 64.389 56.134) (width 1.016) (layer B.Cu) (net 7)))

